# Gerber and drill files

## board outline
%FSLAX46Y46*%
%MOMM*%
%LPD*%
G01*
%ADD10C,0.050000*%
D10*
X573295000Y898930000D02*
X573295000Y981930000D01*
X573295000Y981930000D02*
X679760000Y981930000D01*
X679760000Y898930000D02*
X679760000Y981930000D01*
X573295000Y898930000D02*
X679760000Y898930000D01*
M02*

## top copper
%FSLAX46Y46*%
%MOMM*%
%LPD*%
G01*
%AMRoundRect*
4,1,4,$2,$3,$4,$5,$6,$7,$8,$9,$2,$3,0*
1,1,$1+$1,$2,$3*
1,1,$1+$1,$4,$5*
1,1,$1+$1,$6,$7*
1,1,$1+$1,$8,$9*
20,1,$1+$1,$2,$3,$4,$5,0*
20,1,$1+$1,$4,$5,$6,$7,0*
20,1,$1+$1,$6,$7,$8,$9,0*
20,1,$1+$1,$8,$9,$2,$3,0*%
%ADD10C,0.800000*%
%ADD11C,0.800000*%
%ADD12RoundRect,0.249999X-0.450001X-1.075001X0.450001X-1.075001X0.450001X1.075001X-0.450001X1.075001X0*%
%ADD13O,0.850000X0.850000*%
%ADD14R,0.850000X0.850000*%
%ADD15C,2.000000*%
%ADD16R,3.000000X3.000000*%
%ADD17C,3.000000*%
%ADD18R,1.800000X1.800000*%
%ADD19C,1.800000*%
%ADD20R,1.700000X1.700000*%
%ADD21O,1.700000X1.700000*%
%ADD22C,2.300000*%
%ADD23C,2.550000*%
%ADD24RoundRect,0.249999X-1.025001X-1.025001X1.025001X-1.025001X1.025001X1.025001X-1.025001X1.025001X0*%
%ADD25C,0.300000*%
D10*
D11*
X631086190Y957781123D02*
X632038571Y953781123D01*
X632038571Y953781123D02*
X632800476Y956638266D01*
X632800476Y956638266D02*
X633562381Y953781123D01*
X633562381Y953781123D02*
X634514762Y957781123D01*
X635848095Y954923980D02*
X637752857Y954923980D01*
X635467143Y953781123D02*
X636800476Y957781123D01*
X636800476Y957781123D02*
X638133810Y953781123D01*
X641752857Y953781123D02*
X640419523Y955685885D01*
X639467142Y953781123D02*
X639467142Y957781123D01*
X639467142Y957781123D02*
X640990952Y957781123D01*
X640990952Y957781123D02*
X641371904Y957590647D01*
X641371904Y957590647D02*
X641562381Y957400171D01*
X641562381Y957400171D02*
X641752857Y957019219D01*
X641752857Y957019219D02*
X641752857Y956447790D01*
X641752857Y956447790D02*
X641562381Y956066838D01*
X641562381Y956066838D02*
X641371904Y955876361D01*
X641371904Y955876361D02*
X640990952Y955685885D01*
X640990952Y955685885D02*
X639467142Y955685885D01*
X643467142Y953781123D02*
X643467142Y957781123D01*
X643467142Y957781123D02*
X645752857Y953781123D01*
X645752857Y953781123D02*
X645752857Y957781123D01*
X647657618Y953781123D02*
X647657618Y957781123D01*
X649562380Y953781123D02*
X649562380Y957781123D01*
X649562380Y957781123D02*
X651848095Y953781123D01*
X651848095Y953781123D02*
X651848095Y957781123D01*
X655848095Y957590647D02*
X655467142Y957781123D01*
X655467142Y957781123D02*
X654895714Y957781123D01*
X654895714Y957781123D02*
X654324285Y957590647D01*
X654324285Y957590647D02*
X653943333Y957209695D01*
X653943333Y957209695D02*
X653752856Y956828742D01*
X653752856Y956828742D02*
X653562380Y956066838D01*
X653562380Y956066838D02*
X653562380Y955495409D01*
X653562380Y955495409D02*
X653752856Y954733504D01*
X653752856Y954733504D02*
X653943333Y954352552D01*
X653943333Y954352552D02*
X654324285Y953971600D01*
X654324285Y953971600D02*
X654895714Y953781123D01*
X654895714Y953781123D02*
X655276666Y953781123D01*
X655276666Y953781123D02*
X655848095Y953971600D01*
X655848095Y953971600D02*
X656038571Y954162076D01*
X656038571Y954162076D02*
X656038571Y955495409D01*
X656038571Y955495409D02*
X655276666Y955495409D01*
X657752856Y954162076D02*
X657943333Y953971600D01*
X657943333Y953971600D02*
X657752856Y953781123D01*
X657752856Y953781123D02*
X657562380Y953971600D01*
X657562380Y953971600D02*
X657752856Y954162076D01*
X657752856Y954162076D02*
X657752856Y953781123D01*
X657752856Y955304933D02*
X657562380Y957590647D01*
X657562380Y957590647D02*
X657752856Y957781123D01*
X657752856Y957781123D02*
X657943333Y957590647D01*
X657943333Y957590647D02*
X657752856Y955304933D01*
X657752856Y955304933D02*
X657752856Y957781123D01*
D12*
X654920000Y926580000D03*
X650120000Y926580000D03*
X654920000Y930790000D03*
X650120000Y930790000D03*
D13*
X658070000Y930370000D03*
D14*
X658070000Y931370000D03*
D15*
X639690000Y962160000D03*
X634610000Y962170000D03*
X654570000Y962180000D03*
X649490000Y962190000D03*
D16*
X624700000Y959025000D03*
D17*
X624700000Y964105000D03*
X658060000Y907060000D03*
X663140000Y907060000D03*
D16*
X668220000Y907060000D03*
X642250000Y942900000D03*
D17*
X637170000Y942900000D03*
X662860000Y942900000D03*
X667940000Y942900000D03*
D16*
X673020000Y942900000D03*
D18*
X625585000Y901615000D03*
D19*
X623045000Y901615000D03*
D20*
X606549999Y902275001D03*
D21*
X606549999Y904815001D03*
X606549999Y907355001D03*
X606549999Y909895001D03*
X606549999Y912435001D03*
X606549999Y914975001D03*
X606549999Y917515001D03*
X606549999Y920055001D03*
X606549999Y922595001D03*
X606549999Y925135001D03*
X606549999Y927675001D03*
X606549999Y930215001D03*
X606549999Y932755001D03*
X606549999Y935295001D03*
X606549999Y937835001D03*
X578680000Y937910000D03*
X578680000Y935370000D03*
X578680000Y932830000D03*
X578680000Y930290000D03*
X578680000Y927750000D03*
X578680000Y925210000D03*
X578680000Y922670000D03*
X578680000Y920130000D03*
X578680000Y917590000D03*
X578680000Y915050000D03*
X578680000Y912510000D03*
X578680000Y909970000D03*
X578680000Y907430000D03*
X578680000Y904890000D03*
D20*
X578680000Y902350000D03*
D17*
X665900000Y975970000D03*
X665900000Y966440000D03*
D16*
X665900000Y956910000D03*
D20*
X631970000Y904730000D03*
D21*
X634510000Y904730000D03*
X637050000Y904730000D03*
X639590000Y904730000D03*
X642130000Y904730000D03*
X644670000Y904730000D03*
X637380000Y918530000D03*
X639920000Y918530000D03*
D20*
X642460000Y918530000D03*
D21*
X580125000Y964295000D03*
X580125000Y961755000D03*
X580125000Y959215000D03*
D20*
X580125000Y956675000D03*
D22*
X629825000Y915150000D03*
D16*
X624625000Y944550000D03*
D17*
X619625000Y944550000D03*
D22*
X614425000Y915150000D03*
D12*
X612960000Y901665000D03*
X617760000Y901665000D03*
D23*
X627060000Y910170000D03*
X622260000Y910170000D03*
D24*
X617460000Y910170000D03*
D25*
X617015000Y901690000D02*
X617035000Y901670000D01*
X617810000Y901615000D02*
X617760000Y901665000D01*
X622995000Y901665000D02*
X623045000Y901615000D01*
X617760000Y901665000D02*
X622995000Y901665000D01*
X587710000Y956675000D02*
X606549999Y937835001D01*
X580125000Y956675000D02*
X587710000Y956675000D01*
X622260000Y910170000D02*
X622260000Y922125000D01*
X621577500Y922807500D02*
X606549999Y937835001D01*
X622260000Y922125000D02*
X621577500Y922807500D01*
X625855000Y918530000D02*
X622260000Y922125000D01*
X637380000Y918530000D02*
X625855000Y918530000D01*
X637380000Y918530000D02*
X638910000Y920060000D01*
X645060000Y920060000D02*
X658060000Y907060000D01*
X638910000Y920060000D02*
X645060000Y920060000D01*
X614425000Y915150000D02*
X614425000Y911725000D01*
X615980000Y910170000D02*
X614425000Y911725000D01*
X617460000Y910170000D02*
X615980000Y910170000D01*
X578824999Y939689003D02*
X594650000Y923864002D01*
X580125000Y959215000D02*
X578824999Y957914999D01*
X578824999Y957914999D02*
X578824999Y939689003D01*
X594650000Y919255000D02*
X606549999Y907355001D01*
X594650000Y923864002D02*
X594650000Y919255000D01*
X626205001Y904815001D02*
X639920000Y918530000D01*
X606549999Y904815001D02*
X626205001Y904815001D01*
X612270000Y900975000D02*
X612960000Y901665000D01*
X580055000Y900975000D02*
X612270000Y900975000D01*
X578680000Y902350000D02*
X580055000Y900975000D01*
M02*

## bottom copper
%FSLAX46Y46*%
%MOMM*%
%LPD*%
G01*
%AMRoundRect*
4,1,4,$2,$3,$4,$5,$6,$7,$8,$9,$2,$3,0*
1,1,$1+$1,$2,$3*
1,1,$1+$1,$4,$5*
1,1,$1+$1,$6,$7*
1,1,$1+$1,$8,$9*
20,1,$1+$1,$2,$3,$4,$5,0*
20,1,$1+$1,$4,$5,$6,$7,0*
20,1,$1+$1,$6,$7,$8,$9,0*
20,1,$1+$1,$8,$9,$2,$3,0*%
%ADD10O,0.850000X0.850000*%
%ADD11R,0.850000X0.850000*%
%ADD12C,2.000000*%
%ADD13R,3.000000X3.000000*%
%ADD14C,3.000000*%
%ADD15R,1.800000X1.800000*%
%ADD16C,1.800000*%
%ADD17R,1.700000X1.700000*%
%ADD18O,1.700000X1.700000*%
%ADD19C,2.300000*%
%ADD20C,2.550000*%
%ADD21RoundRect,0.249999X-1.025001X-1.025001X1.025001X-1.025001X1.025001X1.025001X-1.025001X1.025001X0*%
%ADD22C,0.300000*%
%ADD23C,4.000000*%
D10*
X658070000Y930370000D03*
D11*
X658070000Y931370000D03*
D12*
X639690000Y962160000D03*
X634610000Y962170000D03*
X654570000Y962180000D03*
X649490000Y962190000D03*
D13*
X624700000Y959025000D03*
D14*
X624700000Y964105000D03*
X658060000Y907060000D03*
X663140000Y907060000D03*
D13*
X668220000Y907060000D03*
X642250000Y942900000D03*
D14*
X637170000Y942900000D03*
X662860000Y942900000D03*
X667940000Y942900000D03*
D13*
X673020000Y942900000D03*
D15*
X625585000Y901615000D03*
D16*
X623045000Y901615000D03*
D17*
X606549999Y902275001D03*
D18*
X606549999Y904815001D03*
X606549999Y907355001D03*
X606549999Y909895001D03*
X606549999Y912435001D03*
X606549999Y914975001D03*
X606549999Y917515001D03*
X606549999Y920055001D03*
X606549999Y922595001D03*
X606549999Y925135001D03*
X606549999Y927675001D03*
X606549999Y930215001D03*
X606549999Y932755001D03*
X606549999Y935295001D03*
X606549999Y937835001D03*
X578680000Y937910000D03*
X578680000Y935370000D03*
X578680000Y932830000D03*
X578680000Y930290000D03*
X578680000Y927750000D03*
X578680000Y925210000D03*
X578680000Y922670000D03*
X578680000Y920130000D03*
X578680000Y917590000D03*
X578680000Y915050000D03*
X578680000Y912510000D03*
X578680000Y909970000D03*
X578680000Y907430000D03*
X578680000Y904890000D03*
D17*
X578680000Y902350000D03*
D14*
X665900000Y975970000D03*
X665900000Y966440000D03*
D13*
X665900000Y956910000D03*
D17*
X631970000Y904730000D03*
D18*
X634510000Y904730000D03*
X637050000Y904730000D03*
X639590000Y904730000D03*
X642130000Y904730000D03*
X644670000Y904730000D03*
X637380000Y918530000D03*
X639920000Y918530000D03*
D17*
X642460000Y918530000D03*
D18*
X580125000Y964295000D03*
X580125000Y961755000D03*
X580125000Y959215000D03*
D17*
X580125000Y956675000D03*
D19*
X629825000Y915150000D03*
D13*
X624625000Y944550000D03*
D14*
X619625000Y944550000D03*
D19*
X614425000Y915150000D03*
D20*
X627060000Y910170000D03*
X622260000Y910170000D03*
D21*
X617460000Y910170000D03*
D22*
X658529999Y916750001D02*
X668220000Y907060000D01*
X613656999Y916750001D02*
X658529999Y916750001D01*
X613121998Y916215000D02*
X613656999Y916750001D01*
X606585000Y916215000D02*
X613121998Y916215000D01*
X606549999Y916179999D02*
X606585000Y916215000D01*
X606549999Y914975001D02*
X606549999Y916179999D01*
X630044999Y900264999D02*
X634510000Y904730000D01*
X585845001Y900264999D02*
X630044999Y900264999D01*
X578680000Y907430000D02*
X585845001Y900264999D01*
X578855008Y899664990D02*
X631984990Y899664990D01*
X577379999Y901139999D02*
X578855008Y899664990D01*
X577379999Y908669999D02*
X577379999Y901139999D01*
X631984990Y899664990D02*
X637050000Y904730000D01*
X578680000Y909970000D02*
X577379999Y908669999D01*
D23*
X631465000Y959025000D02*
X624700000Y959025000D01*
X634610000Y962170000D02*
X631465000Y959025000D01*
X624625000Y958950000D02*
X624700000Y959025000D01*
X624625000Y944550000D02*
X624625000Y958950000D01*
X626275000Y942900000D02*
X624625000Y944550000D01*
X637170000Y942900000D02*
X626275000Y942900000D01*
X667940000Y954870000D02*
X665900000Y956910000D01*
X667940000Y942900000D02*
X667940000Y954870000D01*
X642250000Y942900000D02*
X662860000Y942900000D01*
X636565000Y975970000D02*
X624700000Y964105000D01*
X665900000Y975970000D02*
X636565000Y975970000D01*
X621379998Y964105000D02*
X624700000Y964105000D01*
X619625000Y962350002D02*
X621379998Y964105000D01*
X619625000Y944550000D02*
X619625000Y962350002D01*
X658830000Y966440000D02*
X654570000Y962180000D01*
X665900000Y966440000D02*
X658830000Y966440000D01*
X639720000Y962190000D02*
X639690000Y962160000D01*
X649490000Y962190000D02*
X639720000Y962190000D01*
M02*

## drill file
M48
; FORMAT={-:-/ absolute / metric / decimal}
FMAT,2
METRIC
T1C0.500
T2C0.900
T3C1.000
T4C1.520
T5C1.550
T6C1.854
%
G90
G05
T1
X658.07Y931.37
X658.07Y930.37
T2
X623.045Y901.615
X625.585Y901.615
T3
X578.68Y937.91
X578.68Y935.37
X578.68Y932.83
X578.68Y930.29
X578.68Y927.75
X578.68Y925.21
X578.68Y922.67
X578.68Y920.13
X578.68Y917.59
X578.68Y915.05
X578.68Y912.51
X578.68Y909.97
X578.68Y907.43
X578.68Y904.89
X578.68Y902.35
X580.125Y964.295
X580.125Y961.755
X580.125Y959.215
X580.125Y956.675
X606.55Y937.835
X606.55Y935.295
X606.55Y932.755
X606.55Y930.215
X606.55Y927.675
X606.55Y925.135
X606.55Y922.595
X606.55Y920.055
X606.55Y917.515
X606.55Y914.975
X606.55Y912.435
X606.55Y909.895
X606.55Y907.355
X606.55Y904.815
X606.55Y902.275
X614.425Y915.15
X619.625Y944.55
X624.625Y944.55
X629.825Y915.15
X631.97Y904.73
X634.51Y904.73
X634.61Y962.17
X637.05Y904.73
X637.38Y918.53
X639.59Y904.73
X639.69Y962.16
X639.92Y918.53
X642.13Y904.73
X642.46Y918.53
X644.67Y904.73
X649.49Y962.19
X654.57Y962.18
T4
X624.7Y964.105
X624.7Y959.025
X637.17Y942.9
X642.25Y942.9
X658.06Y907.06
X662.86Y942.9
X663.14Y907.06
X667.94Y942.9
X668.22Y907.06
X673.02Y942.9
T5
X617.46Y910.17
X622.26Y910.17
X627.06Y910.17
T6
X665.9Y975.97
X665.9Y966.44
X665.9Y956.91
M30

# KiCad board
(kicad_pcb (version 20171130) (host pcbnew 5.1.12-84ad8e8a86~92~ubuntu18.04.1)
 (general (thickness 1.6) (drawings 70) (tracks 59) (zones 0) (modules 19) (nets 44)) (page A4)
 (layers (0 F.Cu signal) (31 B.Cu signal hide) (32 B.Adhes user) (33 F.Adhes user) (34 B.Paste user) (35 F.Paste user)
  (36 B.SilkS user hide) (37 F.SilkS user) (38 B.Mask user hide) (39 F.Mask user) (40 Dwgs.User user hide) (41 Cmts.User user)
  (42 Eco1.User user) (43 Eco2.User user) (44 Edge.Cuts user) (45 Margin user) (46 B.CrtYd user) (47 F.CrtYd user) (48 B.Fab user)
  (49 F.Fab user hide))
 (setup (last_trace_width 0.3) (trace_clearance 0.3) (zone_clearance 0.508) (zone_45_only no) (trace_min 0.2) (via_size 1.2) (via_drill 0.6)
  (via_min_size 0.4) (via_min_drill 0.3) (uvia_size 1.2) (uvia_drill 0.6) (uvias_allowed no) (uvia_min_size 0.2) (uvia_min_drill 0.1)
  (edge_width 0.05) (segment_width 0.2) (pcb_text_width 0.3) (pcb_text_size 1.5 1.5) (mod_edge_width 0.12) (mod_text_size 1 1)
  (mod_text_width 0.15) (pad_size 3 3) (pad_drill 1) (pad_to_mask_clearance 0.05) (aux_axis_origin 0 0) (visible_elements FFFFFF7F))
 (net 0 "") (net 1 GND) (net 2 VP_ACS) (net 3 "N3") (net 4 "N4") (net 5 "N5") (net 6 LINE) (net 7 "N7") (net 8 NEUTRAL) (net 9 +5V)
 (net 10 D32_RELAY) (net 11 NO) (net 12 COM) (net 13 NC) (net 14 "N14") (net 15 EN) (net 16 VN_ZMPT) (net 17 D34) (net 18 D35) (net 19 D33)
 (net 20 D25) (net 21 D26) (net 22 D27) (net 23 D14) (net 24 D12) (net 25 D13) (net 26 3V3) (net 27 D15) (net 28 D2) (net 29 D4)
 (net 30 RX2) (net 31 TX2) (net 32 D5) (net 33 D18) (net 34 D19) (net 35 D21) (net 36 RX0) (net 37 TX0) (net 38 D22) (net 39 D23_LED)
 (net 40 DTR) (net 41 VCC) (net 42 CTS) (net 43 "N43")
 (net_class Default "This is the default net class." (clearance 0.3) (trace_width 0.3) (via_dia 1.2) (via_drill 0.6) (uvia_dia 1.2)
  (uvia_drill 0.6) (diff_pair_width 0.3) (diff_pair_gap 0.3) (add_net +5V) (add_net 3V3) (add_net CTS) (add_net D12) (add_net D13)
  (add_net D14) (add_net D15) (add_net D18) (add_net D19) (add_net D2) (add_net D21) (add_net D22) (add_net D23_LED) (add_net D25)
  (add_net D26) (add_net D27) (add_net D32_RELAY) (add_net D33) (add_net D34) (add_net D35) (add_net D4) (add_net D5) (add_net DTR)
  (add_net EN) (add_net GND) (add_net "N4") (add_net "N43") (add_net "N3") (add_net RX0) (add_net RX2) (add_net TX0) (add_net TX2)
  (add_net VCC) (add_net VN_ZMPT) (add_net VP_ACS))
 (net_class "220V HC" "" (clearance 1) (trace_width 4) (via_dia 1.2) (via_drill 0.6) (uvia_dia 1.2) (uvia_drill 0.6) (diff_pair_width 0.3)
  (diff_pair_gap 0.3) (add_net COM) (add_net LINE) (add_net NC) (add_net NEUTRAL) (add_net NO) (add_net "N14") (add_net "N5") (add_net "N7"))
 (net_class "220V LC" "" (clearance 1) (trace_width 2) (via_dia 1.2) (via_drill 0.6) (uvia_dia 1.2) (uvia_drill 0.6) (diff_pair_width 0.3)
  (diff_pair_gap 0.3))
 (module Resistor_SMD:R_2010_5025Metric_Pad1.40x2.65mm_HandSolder (layer F.Cu) (at 652.52 -926.58)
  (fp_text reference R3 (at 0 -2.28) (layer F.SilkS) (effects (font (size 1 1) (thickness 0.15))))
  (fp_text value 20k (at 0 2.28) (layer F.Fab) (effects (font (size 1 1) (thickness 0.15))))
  (pad 2 smd roundrect (at 2.4 0) (size 1.4 2.65) (layers F.Cu F.Paste F.Mask) (roundrect_rratio 0.178571) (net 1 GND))
  (pad 1 smd roundrect (at -2.4 0) (size 1.4 2.65) (layers F.Cu F.Paste F.Mask) (roundrect_rratio 0.178571) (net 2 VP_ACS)))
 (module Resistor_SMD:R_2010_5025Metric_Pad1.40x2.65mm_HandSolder (layer F.Cu) (at 652.52 -930.79)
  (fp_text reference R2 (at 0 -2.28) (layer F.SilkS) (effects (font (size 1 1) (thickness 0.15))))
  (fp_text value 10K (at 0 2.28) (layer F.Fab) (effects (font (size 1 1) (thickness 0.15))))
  (pad 2 smd roundrect (at 2.4 0) (size 1.4 2.65) (layers F.Cu F.Paste F.Mask) (roundrect_rratio 0.178571) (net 2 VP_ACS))
  (pad 1 smd roundrect (at -2.4 0) (size 1.4 2.65) (layers F.Cu F.Paste F.Mask) (roundrect_rratio 0.178571) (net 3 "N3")))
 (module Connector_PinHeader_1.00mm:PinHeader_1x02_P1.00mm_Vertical (layer F.Cu) (at 658.07 -931.37)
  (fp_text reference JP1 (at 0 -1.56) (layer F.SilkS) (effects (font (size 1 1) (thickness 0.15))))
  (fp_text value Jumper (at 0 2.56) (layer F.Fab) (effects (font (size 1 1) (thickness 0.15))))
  (pad 2 thru_hole oval (at 0 1) (size 0.85 0.85) (drill 0.5) (layers *.Cu *.Mask) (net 3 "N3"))
  (pad 1 thru_hole rect (at 0 0) (size 0.85 0.85) (drill 0.5) (layers *.Cu *.Mask) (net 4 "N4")))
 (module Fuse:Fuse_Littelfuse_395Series (layer F.Cu) (at 634.61 -962.17)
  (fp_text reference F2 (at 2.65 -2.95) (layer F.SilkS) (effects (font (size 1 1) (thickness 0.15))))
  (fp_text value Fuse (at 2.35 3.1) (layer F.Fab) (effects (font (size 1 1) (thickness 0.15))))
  (pad 2 thru_hole circle (at 5.08 0.01) (size 2 2) (drill 1) (layers *.Cu *.Mask) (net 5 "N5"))
  (pad 1 thru_hole circle (at 0 0) (size 2 2) (drill 1) (layers *.Cu *.Mask) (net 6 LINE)))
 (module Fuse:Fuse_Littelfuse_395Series (layer F.Cu) (at 649.49 -962.19)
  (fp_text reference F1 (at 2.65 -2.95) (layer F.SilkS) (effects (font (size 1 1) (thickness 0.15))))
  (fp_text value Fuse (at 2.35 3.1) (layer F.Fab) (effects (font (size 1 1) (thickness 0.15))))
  (pad 2 thru_hole circle (at 5.08 0.01) (size 2 2) (drill 1) (layers *.Cu *.Mask) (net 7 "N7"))
  (pad 1 thru_hole circle (at 0 0) (size 2 2) (drill 1) (layers *.Cu *.Mask) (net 5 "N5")))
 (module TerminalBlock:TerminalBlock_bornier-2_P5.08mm (layer F.Cu) (at 624.7 -959.025 90)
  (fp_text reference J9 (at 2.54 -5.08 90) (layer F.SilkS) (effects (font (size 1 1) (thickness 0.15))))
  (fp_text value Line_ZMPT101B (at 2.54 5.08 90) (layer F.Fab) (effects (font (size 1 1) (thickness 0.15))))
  (pad 1 thru_hole rect (at 0 0 90) (size 3 3) (drill 1.52) (layers *.Cu *.Mask) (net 6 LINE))
  (pad 2 thru_hole circle (at 5.08 0 90) (size 3 3) (drill 1.52) (layers *.Cu *.Mask) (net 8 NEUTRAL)))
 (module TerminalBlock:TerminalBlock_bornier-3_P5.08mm (layer F.Cu) (at 668.22 -907.06 180)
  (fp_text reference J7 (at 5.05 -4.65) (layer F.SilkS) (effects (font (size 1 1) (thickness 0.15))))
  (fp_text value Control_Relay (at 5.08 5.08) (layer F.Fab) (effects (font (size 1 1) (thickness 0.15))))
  (pad 3 thru_hole circle (at 10.16 0 180) (size 3 3) (drill 1.52) (layers *.Cu *.Mask) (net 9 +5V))
  (pad 2 thru_hole circle (at 5.08 0 180) (size 3 3) (drill 1.52) (layers *.Cu *.Mask) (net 1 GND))
  (pad 1 thru_hole rect (at 0 0 180) (size 3 3) (drill 1.52) (layers *.Cu *.Mask) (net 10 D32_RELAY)))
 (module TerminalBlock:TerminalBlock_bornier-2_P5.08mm (layer F.Cu) (at 642.25 -942.9 180)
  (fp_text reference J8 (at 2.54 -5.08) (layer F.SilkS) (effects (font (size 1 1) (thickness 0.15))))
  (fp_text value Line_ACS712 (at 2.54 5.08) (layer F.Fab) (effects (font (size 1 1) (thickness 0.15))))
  (pad 1 thru_hole rect (at 0 0 180) (size 3 3) (drill 1.52) (layers *.Cu *.Mask) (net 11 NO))
  (pad 2 thru_hole circle (at 5.08 0 180) (size 3 3) (drill 1.52) (layers *.Cu *.Mask) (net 6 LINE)))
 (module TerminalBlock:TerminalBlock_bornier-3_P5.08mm (layer F.Cu) (at 673.02 -942.9 180)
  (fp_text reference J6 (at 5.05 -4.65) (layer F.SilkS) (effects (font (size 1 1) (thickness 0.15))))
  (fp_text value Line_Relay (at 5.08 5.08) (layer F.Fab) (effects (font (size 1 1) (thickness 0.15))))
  (pad 3 thru_hole circle (at 10.16 0 180) (size 3 3) (drill 1.52) (layers *.Cu *.Mask) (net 11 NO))
  (pad 2 thru_hole circle (at 5.08 0 180) (size 3 3) (drill 1.52) (layers *.Cu *.Mask) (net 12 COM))
  (pad 1 thru_hole rect (at 0 0 180) (size 3 3) (drill 1.52) (layers *.Cu *.Mask) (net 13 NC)))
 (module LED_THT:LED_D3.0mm (layer F.Cu) (at 625.585 -901.615 180)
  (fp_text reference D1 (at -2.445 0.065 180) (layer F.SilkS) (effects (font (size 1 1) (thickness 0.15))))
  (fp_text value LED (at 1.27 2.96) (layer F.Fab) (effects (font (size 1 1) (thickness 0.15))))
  (pad 1 thru_hole rect (at 0 0 180) (size 1.8 1.8) (drill 0.9) (layers *.Cu *.Mask) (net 1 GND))
  (pad 2 thru_hole circle (at 2.54 0 180) (size 1.8 1.8) (drill 0.9) (layers *.Cu *.Mask) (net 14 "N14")))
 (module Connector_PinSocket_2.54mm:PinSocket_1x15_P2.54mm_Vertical (layer F.Cu) (at 606.549999 -902.275001 180)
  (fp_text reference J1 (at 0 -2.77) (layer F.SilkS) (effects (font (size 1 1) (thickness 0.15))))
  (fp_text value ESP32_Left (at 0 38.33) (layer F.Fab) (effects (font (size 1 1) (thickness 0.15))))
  (pad 1 thru_hole rect (at 0 0 180) (size 1.7 1.7) (drill 1) (layers *.Cu *.Mask) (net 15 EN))
  (pad 2 thru_hole oval (at 0 2.54 180) (size 1.7 1.7) (drill 1) (layers *.Cu *.Mask) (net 2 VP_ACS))
  (pad 3 thru_hole oval (at 0 5.08 180) (size 1.7 1.7) (drill 1) (layers *.Cu *.Mask) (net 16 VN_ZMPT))
  (pad 4 thru_hole oval (at 0 7.62 180) (size 1.7 1.7) (drill 1) (layers *.Cu *.Mask) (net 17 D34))
  (pad 5 thru_hole oval (at 0 10.16 180) (size 1.7 1.7) (drill 1) (layers *.Cu *.Mask) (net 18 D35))
  (pad 6 thru_hole oval (at 0 12.7 180) (size 1.7 1.7) (drill 1) (layers *.Cu *.Mask) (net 10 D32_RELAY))
  (pad 7 thru_hole oval (at 0 15.24 180) (size 1.7 1.7) (drill 1) (layers *.Cu *.Mask) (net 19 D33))
  (pad 8 thru_hole oval (at 0 17.78 180) (size 1.7 1.7) (drill 1) (layers *.Cu *.Mask) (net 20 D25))
  (pad 9 thru_hole oval (at 0 20.32 180) (size 1.7 1.7) (drill 1) (layers *.Cu *.Mask) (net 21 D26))
  (pad 10 thru_hole oval (at 0 22.86 180) (size 1.7 1.7) (drill 1) (layers *.Cu *.Mask) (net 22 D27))
  (pad 11 thru_hole oval (at 0 25.4 180) (size 1.7 1.7) (drill 1) (layers *.Cu *.Mask) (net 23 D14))
  (pad 12 thru_hole oval (at 0 27.94 180) (size 1.7 1.7) (drill 1) (layers *.Cu *.Mask) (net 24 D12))
  (pad 13 thru_hole oval (at 0 30.48 180) (size 1.7 1.7) (drill 1) (layers *.Cu *.Mask) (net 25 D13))
  (pad 14 thru_hole oval (at 0 33.02 180) (size 1.7 1.7) (drill 1) (layers *.Cu *.Mask) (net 1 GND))
  (pad 15 thru_hole oval (at 0 35.56 180) (size 1.7 1.7) (drill 1) (layers *.Cu *.Mask) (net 9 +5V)))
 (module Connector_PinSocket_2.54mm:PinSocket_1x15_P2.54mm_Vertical (layer F.Cu) (at 578.68 -902.35 180)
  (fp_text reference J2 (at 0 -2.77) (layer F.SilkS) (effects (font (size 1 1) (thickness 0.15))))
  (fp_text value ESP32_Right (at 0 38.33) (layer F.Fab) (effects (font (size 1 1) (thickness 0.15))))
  (pad 15 thru_hole oval (at 0 35.56 180) (size 1.7 1.7) (drill 1) (layers *.Cu *.Mask) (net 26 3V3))
  (pad 14 thru_hole oval (at 0 33.02 180) (size 1.7 1.7) (drill 1) (layers *.Cu *.Mask) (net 1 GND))
  (pad 13 thru_hole oval (at 0 30.48 180) (size 1.7 1.7) (drill 1) (layers *.Cu *.Mask) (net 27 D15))
  (pad 12 thru_hole oval (at 0 27.94 180) (size 1.7 1.7) (drill 1) (layers *.Cu *.Mask) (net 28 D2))
  (pad 11 thru_hole oval (at 0 25.4 180) (size 1.7 1.7) (drill 1) (layers *.Cu *.Mask) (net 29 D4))
  (pad 10 thru_hole oval (at 0 22.86 180) (size 1.7 1.7) (drill 1) (layers *.Cu *.Mask) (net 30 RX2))
  (pad 9 thru_hole oval (at 0 20.32 180) (size 1.7 1.7) (drill 1) (layers *.Cu *.Mask) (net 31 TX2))
  (pad 8 thru_hole oval (at 0 17.78 180) (size 1.7 1.7) (drill 1) (layers *.Cu *.Mask) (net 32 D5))
  (pad 7 thru_hole oval (at 0 15.24 180) (size 1.7 1.7) (drill 1) (layers *.Cu *.Mask) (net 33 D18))
  (pad 6 thru_hole oval (at 0 12.7 180) (size 1.7 1.7) (drill 1) (layers *.Cu *.Mask) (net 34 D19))
  (pad 5 thru_hole oval (at 0 10.16 180) (size 1.7 1.7) (drill 1) (layers *.Cu *.Mask) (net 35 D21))
  (pad 4 thru_hole oval (at 0 7.62 180) (size 1.7 1.7) (drill 1) (layers *.Cu *.Mask) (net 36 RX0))
  (pad 3 thru_hole oval (at 0 5.08 180) (size 1.7 1.7) (drill 1) (layers *.Cu *.Mask) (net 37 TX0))
  (pad 2 thru_hole oval (at 0 2.54 180) (size 1.7 1.7) (drill 1) (layers *.Cu *.Mask) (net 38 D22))
  (pad 1 thru_hole rect (at 0 0 180) (size 1.7 1.7) (drill 1) (layers *.Cu *.Mask) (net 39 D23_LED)))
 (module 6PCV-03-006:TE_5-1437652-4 (layer F.Cu) (at 665.9 -956.91 90)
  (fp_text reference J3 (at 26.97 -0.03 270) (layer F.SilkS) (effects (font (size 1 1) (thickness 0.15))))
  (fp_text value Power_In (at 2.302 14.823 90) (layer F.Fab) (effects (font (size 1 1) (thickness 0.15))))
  (pad 3 thru_hole circle (at 19.06 0 90) (size 3 3) (drill 1.854) (layers *.Cu *.Mask) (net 8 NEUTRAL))
  (pad 2 thru_hole circle (at 9.53 0 90) (size 3 3) (drill 1.854) (layers *.Cu *.Mask) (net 7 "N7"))
  (pad 1 thru_hole rect (at 0 0 90) (size 3 3) (drill 1.854) (layers *.Cu *.Mask) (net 12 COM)))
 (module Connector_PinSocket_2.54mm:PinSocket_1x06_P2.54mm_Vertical (layer F.Cu) (at 631.97 -904.73 90)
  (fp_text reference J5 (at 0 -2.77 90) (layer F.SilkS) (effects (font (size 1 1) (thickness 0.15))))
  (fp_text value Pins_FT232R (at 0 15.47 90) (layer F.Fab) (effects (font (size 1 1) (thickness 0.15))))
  (pad 1 thru_hole rect (at 0 0 90) (size 1.7 1.7) (drill 1) (layers *.Cu *.Mask) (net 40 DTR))
  (pad 2 thru_hole oval (at 0 2.54 90) (size 1.7 1.7) (drill 1) (layers *.Cu *.Mask) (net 37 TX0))
  (pad 3 thru_hole oval (at 0 5.08 90) (size 1.7 1.7) (drill 1) (layers *.Cu *.Mask) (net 36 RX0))
  (pad 4 thru_hole oval (at 0 7.62 90) (size 1.7 1.7) (drill 1) (layers *.Cu *.Mask) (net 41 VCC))
  (pad 5 thru_hole oval (at 0 10.16 90) (size 1.7 1.7) (drill 1) (layers *.Cu *.Mask) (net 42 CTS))
  (pad 6 thru_hole oval (at 0 12.7 90) (size 1.7 1.7) (drill 1) (layers *.Cu *.Mask) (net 1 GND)))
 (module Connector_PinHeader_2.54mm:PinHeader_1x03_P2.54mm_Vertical (layer F.Cu) (at 642.46 -918.53 270)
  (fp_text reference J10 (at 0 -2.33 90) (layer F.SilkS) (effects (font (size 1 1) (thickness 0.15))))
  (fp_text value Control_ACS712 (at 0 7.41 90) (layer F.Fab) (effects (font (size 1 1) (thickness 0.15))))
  (pad 3 thru_hole oval (at 0 5.08 270) (size 1.7 1.7) (drill 1) (layers *.Cu *.Mask) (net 9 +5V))
  (pad 2 thru_hole oval (at 0 2.54 270) (size 1.7 1.7) (drill 1) (layers *.Cu *.Mask) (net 4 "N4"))
  (pad 1 thru_hole rect (at 0 0 270) (size 1.7 1.7) (drill 1) (layers *.Cu *.Mask) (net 1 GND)))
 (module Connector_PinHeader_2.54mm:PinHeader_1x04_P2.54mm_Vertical (layer F.Cu) (at 580.125 -956.675 180)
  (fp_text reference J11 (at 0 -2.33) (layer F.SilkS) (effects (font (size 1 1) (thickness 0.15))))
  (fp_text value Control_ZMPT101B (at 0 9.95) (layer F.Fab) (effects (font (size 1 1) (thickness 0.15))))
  (pad 4 thru_hole oval (at 0 7.62 180) (size 1.7 1.7) (drill 1) (layers *.Cu *.Mask) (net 1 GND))
  (pad 3 thru_hole oval (at 0 5.08 180) (size 1.7 1.7) (drill 1) (layers *.Cu *.Mask) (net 1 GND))
  (pad 2 thru_hole oval (at 0 2.54 180) (size 1.7 1.7) (drill 1) (layers *.Cu *.Mask) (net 16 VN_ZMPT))
  (pad 1 thru_hole rect (at 0 0 180) (size 1.7 1.7) (drill 1) (layers *.Cu *.Mask) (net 9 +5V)))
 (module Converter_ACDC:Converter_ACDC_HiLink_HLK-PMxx (layer F.Cu) (at 624.625 -944.55 270)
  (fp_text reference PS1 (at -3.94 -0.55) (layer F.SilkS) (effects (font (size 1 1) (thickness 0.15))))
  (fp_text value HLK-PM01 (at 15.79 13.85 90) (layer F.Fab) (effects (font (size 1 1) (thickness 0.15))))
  (pad 3 thru_hole circle (at 29.4 -5.2 270) (size 2.3 2.3) (drill 1) (layers *.Cu *.Mask) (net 1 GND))
  (pad 1 thru_hole rect (at 0 0 270) (size 3 3) (drill 1) (layers *.Cu *.Mask) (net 6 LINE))
  (pad 2 thru_hole circle (at 0 5 270) (size 3 3) (drill 1) (layers *.Cu *.Mask) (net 8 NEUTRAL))
  (pad 4 thru_hole circle (at 29.4 10.2 270) (size 2.3 2.3) (drill 1) (layers *.Cu *.Mask) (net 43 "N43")))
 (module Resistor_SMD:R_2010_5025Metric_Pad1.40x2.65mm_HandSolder (layer F.Cu) (at 615.36 -901.665)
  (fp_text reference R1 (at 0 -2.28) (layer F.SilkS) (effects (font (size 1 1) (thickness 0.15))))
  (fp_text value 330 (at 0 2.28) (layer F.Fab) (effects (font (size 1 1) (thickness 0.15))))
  (pad 1 smd roundrect (at -2.4 0) (size 1.4 2.65) (layers F.Cu F.Paste F.Mask) (roundrect_rratio 0.178571) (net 39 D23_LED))
  (pad 2 smd roundrect (at 2.4 0) (size 1.4 2.65) (layers F.Cu F.Paste F.Mask) (roundrect_rratio 0.178571) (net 14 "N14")))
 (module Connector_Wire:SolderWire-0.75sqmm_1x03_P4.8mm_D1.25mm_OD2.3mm (layer F.Cu) (at 617.46 -910.17)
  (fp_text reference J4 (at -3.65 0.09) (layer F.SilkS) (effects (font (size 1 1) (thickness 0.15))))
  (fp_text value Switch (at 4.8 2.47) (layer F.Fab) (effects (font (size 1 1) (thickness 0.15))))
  (pad 3 thru_hole circle (at 9.6 0) (size 2.55 2.55) (drill 1.55) (layers *.Cu *.Mask) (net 1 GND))
  (pad 2 thru_hole circle (at 4.8 0) (size 2.55 2.55) (drill 1.55) (layers *.Cu *.Mask) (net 9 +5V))
  (pad 1 thru_hole roundrect (at 0 0) (size 2.55 2.55) (drill 1.55) (layers *.Cu *.Mask) (roundrect_rratio 0.098039) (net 43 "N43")))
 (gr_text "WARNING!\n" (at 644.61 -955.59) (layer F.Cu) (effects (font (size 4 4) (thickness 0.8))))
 (gr_line (start 573.295 -898.93) (end 573.295 -981.93) (layer Edge.Cuts) (width 0.05))
 (gr_line (start 573.295 -981.93) (end 679.76 -981.93) (layer Edge.Cuts) (width 0.05))
 (gr_line (start 679.76 -898.93) (end 679.76 -981.93) (layer Edge.Cuts) (width 0.05))
 (gr_line (start 573.295 -898.93) (end 679.76 -898.93) (layer Edge.Cuts) (width 0.05))
 (segment (start 617.015 -901.69) (end 617.035 -901.67) (width 0.3) (layer F.Cu) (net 14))
 (segment (start 617.81 -901.615) (end 617.76 -901.665) (width 0.3) (layer F.Cu) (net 14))
 (segment (start 622.995 -901.665) (end 623.045 -901.615) (width 0.3) (layer F.Cu) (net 14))
 (segment (start 617.76 -901.665) (end 622.995 -901.665) (width 0.3) (layer F.Cu) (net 14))
 (segment (start 587.71 -956.675) (end 606.549999 -937.835001) (width 0.3) (layer F.Cu) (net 9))
 (segment (start 580.125 -956.675) (end 587.71 -956.675) (width 0.3) (layer F.Cu) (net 9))
 (segment (start 622.26 -910.17) (end 622.26 -922.125) (width 0.3) (layer F.Cu) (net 9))
 (segment (start 621.5775 -922.8075) (end 606.549999 -937.835001) (width 0.3) (layer F.Cu) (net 9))
 (segment (start 622.26 -922.125) (end 621.5775 -922.8075) (width 0.3) (layer F.Cu) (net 9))
 (segment (start 625.855 -918.53) (end 622.26 -922.125) (width 0.3) (layer F.Cu) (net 9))
 (segment (start 637.38 -918.53) (end 625.855 -918.53) (width 0.3) (layer F.Cu) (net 9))
 (segment (start 637.38 -918.53) (end 638.91 -920.06) (width 0.3) (layer F.Cu) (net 9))
 (segment (start 645.06 -920.06) (end 658.06 -907.06) (width 0.3) (layer F.Cu) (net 9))
 (segment (start 638.91 -920.06) (end 645.06 -920.06) (width 0.3) (layer F.Cu) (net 9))
 (segment (start 658.529999 -916.750001) (end 668.22 -907.06) (width 0.3) (layer B.Cu) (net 10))
 (segment (start 613.656999 -916.750001) (end 658.529999 -916.750001) (width 0.3) (layer B.Cu) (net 10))
 (segment (start 613.121998 -916.215) (end 613.656999 -916.750001) (width 0.3) (layer B.Cu) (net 10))
 (segment (start 606.585 -916.215) (end 613.121998 -916.215) (width 0.3) (layer B.Cu) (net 10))
 (segment (start 606.549999 -916.179999) (end 606.585 -916.215) (width 0.3) (layer B.Cu) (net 10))
 (segment (start 606.549999 -914.975001) (end 606.549999 -916.179999) (width 0.3) (layer B.Cu) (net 10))
 (segment (start 630.044999 -900.264999) (end 634.51 -904.73) (width 0.3) (layer B.Cu) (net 37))
 (segment (start 585.845001 -900.264999) (end 630.044999 -900.264999) (width 0.3) (layer B.Cu) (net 37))
 (segment (start 578.68 -907.43) (end 585.845001 -900.264999) (width 0.3) (layer B.Cu) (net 37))
 (segment (start 578.855008 -899.66499) (end 631.98499 -899.66499) (width 0.3) (layer B.Cu) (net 36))
 (segment (start 577.379999 -901.139999) (end 578.855008 -899.66499) (width 0.3) (layer B.Cu) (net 36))
 (segment (start 577.379999 -908.669999) (end 577.379999 -901.139999) (width 0.3) (layer B.Cu) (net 36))
 (segment (start 631.98499 -899.66499) (end 637.05 -904.73) (width 0.3) (layer B.Cu) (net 36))
 (segment (start 578.68 -909.97) (end 577.379999 -908.669999) (width 0.3) (layer B.Cu) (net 36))
 (segment (start 631.465 -959.025) (end 624.7 -959.025) (width 4) (layer B.Cu) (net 6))
 (segment (start 634.61 -962.17) (end 631.465 -959.025) (width 4) (layer B.Cu) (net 6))
 (segment (start 624.625 -958.95) (end 624.7 -959.025) (width 4) (layer B.Cu) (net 6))
 (segment (start 624.625 -944.55) (end 624.625 -958.95) (width 4) (layer B.Cu) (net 6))
 (segment (start 626.275 -942.9) (end 624.625 -944.55) (width 4) (layer B.Cu) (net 6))
 (segment (start 637.17 -942.9) (end 626.275 -942.9) (width 4) (layer B.Cu) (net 6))
 (segment (start 667.94 -954.87) (end 665.9 -956.91) (width 4) (layer B.Cu) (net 12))
 (segment (start 667.94 -942.9) (end 667.94 -954.87) (width 4) (layer B.Cu) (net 12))
 (segment (start 642.25 -942.9) (end 662.86 -942.9) (width 4) (layer B.Cu) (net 11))
 (segment (start 614.425 -915.15) (end 614.425 -911.725) (width 0.3) (layer F.Cu) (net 43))
 (segment (start 615.98 -910.17) (end 614.425 -911.725) (width 0.3) (layer F.Cu) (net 43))
 (segment (start 617.46 -910.17) (end 615.98 -910.17) (width 0.3) (layer F.Cu) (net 43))
 (segment (start 578.824999 -939.689003) (end 594.65 -923.864002) (width 0.3) (layer F.Cu) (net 16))
 (segment (start 580.125 -959.215) (end 578.824999 -957.914999) (width 0.3) (layer F.Cu) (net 16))
 (segment (start 578.824999 -957.914999) (end 578.824999 -939.689003) (width 0.3) (layer F.Cu) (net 16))
 (segment (start 594.65 -919.255) (end 606.549999 -907.355001) (width 0.3) (layer F.Cu) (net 16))
 (segment (start 594.65 -923.864002) (end 594.65 -919.255) (width 0.3) (layer F.Cu) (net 16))
 (segment (start 626.205001 -904.815001) (end 639.92 -918.53) (width 0.3) (layer F.Cu) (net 2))
 (segment (start 606.549999 -904.815001) (end 626.205001 -904.815001) (width 0.3) (layer F.Cu) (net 2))
 (segment (start 612.27 -900.975) (end 612.96 -901.665) (width 0.3) (layer F.Cu) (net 39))
 (segment (start 580.055 -900.975) (end 612.27 -900.975) (width 0.3) (layer F.Cu) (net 39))
 (segment (start 578.68 -902.35) (end 580.055 -900.975) (width 0.3) (layer F.Cu) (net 39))
 (segment (start 636.565 -975.97) (end 624.7 -964.105) (width 4) (layer B.Cu) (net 8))
 (segment (start 665.9 -975.97) (end 636.565 -975.97) (width 4) (layer B.Cu) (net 8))
 (segment (start 621.379998 -964.105) (end 624.7 -964.105) (width 4) (layer B.Cu) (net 8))
 (segment (start 619.625 -962.350002) (end 621.379998 -964.105) (width 4) (layer B.Cu) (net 8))
 (segment (start 619.625 -944.55) (end 619.625 -962.350002) (width 4) (layer B.Cu) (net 8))
 (segment (start 658.83 -966.44) (end 654.57 -962.18) (width 4) (layer B.Cu) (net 7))
 (segment (start 665.9 -966.44) (end 658.83 -966.44) (width 4) (layer B.Cu) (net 7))
 (segment (start 639.72 -962.19) (end 639.69 -962.16) (width 4) (layer B.Cu) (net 5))
 (segment (start 649.49 -962.19) (end 639.72 -962.19) (width 4) (layer B.Cu) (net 5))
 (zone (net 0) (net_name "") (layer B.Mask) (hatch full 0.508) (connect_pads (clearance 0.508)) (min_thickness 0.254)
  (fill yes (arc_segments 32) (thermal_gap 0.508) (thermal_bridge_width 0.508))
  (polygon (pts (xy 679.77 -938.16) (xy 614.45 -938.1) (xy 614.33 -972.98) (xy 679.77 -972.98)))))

